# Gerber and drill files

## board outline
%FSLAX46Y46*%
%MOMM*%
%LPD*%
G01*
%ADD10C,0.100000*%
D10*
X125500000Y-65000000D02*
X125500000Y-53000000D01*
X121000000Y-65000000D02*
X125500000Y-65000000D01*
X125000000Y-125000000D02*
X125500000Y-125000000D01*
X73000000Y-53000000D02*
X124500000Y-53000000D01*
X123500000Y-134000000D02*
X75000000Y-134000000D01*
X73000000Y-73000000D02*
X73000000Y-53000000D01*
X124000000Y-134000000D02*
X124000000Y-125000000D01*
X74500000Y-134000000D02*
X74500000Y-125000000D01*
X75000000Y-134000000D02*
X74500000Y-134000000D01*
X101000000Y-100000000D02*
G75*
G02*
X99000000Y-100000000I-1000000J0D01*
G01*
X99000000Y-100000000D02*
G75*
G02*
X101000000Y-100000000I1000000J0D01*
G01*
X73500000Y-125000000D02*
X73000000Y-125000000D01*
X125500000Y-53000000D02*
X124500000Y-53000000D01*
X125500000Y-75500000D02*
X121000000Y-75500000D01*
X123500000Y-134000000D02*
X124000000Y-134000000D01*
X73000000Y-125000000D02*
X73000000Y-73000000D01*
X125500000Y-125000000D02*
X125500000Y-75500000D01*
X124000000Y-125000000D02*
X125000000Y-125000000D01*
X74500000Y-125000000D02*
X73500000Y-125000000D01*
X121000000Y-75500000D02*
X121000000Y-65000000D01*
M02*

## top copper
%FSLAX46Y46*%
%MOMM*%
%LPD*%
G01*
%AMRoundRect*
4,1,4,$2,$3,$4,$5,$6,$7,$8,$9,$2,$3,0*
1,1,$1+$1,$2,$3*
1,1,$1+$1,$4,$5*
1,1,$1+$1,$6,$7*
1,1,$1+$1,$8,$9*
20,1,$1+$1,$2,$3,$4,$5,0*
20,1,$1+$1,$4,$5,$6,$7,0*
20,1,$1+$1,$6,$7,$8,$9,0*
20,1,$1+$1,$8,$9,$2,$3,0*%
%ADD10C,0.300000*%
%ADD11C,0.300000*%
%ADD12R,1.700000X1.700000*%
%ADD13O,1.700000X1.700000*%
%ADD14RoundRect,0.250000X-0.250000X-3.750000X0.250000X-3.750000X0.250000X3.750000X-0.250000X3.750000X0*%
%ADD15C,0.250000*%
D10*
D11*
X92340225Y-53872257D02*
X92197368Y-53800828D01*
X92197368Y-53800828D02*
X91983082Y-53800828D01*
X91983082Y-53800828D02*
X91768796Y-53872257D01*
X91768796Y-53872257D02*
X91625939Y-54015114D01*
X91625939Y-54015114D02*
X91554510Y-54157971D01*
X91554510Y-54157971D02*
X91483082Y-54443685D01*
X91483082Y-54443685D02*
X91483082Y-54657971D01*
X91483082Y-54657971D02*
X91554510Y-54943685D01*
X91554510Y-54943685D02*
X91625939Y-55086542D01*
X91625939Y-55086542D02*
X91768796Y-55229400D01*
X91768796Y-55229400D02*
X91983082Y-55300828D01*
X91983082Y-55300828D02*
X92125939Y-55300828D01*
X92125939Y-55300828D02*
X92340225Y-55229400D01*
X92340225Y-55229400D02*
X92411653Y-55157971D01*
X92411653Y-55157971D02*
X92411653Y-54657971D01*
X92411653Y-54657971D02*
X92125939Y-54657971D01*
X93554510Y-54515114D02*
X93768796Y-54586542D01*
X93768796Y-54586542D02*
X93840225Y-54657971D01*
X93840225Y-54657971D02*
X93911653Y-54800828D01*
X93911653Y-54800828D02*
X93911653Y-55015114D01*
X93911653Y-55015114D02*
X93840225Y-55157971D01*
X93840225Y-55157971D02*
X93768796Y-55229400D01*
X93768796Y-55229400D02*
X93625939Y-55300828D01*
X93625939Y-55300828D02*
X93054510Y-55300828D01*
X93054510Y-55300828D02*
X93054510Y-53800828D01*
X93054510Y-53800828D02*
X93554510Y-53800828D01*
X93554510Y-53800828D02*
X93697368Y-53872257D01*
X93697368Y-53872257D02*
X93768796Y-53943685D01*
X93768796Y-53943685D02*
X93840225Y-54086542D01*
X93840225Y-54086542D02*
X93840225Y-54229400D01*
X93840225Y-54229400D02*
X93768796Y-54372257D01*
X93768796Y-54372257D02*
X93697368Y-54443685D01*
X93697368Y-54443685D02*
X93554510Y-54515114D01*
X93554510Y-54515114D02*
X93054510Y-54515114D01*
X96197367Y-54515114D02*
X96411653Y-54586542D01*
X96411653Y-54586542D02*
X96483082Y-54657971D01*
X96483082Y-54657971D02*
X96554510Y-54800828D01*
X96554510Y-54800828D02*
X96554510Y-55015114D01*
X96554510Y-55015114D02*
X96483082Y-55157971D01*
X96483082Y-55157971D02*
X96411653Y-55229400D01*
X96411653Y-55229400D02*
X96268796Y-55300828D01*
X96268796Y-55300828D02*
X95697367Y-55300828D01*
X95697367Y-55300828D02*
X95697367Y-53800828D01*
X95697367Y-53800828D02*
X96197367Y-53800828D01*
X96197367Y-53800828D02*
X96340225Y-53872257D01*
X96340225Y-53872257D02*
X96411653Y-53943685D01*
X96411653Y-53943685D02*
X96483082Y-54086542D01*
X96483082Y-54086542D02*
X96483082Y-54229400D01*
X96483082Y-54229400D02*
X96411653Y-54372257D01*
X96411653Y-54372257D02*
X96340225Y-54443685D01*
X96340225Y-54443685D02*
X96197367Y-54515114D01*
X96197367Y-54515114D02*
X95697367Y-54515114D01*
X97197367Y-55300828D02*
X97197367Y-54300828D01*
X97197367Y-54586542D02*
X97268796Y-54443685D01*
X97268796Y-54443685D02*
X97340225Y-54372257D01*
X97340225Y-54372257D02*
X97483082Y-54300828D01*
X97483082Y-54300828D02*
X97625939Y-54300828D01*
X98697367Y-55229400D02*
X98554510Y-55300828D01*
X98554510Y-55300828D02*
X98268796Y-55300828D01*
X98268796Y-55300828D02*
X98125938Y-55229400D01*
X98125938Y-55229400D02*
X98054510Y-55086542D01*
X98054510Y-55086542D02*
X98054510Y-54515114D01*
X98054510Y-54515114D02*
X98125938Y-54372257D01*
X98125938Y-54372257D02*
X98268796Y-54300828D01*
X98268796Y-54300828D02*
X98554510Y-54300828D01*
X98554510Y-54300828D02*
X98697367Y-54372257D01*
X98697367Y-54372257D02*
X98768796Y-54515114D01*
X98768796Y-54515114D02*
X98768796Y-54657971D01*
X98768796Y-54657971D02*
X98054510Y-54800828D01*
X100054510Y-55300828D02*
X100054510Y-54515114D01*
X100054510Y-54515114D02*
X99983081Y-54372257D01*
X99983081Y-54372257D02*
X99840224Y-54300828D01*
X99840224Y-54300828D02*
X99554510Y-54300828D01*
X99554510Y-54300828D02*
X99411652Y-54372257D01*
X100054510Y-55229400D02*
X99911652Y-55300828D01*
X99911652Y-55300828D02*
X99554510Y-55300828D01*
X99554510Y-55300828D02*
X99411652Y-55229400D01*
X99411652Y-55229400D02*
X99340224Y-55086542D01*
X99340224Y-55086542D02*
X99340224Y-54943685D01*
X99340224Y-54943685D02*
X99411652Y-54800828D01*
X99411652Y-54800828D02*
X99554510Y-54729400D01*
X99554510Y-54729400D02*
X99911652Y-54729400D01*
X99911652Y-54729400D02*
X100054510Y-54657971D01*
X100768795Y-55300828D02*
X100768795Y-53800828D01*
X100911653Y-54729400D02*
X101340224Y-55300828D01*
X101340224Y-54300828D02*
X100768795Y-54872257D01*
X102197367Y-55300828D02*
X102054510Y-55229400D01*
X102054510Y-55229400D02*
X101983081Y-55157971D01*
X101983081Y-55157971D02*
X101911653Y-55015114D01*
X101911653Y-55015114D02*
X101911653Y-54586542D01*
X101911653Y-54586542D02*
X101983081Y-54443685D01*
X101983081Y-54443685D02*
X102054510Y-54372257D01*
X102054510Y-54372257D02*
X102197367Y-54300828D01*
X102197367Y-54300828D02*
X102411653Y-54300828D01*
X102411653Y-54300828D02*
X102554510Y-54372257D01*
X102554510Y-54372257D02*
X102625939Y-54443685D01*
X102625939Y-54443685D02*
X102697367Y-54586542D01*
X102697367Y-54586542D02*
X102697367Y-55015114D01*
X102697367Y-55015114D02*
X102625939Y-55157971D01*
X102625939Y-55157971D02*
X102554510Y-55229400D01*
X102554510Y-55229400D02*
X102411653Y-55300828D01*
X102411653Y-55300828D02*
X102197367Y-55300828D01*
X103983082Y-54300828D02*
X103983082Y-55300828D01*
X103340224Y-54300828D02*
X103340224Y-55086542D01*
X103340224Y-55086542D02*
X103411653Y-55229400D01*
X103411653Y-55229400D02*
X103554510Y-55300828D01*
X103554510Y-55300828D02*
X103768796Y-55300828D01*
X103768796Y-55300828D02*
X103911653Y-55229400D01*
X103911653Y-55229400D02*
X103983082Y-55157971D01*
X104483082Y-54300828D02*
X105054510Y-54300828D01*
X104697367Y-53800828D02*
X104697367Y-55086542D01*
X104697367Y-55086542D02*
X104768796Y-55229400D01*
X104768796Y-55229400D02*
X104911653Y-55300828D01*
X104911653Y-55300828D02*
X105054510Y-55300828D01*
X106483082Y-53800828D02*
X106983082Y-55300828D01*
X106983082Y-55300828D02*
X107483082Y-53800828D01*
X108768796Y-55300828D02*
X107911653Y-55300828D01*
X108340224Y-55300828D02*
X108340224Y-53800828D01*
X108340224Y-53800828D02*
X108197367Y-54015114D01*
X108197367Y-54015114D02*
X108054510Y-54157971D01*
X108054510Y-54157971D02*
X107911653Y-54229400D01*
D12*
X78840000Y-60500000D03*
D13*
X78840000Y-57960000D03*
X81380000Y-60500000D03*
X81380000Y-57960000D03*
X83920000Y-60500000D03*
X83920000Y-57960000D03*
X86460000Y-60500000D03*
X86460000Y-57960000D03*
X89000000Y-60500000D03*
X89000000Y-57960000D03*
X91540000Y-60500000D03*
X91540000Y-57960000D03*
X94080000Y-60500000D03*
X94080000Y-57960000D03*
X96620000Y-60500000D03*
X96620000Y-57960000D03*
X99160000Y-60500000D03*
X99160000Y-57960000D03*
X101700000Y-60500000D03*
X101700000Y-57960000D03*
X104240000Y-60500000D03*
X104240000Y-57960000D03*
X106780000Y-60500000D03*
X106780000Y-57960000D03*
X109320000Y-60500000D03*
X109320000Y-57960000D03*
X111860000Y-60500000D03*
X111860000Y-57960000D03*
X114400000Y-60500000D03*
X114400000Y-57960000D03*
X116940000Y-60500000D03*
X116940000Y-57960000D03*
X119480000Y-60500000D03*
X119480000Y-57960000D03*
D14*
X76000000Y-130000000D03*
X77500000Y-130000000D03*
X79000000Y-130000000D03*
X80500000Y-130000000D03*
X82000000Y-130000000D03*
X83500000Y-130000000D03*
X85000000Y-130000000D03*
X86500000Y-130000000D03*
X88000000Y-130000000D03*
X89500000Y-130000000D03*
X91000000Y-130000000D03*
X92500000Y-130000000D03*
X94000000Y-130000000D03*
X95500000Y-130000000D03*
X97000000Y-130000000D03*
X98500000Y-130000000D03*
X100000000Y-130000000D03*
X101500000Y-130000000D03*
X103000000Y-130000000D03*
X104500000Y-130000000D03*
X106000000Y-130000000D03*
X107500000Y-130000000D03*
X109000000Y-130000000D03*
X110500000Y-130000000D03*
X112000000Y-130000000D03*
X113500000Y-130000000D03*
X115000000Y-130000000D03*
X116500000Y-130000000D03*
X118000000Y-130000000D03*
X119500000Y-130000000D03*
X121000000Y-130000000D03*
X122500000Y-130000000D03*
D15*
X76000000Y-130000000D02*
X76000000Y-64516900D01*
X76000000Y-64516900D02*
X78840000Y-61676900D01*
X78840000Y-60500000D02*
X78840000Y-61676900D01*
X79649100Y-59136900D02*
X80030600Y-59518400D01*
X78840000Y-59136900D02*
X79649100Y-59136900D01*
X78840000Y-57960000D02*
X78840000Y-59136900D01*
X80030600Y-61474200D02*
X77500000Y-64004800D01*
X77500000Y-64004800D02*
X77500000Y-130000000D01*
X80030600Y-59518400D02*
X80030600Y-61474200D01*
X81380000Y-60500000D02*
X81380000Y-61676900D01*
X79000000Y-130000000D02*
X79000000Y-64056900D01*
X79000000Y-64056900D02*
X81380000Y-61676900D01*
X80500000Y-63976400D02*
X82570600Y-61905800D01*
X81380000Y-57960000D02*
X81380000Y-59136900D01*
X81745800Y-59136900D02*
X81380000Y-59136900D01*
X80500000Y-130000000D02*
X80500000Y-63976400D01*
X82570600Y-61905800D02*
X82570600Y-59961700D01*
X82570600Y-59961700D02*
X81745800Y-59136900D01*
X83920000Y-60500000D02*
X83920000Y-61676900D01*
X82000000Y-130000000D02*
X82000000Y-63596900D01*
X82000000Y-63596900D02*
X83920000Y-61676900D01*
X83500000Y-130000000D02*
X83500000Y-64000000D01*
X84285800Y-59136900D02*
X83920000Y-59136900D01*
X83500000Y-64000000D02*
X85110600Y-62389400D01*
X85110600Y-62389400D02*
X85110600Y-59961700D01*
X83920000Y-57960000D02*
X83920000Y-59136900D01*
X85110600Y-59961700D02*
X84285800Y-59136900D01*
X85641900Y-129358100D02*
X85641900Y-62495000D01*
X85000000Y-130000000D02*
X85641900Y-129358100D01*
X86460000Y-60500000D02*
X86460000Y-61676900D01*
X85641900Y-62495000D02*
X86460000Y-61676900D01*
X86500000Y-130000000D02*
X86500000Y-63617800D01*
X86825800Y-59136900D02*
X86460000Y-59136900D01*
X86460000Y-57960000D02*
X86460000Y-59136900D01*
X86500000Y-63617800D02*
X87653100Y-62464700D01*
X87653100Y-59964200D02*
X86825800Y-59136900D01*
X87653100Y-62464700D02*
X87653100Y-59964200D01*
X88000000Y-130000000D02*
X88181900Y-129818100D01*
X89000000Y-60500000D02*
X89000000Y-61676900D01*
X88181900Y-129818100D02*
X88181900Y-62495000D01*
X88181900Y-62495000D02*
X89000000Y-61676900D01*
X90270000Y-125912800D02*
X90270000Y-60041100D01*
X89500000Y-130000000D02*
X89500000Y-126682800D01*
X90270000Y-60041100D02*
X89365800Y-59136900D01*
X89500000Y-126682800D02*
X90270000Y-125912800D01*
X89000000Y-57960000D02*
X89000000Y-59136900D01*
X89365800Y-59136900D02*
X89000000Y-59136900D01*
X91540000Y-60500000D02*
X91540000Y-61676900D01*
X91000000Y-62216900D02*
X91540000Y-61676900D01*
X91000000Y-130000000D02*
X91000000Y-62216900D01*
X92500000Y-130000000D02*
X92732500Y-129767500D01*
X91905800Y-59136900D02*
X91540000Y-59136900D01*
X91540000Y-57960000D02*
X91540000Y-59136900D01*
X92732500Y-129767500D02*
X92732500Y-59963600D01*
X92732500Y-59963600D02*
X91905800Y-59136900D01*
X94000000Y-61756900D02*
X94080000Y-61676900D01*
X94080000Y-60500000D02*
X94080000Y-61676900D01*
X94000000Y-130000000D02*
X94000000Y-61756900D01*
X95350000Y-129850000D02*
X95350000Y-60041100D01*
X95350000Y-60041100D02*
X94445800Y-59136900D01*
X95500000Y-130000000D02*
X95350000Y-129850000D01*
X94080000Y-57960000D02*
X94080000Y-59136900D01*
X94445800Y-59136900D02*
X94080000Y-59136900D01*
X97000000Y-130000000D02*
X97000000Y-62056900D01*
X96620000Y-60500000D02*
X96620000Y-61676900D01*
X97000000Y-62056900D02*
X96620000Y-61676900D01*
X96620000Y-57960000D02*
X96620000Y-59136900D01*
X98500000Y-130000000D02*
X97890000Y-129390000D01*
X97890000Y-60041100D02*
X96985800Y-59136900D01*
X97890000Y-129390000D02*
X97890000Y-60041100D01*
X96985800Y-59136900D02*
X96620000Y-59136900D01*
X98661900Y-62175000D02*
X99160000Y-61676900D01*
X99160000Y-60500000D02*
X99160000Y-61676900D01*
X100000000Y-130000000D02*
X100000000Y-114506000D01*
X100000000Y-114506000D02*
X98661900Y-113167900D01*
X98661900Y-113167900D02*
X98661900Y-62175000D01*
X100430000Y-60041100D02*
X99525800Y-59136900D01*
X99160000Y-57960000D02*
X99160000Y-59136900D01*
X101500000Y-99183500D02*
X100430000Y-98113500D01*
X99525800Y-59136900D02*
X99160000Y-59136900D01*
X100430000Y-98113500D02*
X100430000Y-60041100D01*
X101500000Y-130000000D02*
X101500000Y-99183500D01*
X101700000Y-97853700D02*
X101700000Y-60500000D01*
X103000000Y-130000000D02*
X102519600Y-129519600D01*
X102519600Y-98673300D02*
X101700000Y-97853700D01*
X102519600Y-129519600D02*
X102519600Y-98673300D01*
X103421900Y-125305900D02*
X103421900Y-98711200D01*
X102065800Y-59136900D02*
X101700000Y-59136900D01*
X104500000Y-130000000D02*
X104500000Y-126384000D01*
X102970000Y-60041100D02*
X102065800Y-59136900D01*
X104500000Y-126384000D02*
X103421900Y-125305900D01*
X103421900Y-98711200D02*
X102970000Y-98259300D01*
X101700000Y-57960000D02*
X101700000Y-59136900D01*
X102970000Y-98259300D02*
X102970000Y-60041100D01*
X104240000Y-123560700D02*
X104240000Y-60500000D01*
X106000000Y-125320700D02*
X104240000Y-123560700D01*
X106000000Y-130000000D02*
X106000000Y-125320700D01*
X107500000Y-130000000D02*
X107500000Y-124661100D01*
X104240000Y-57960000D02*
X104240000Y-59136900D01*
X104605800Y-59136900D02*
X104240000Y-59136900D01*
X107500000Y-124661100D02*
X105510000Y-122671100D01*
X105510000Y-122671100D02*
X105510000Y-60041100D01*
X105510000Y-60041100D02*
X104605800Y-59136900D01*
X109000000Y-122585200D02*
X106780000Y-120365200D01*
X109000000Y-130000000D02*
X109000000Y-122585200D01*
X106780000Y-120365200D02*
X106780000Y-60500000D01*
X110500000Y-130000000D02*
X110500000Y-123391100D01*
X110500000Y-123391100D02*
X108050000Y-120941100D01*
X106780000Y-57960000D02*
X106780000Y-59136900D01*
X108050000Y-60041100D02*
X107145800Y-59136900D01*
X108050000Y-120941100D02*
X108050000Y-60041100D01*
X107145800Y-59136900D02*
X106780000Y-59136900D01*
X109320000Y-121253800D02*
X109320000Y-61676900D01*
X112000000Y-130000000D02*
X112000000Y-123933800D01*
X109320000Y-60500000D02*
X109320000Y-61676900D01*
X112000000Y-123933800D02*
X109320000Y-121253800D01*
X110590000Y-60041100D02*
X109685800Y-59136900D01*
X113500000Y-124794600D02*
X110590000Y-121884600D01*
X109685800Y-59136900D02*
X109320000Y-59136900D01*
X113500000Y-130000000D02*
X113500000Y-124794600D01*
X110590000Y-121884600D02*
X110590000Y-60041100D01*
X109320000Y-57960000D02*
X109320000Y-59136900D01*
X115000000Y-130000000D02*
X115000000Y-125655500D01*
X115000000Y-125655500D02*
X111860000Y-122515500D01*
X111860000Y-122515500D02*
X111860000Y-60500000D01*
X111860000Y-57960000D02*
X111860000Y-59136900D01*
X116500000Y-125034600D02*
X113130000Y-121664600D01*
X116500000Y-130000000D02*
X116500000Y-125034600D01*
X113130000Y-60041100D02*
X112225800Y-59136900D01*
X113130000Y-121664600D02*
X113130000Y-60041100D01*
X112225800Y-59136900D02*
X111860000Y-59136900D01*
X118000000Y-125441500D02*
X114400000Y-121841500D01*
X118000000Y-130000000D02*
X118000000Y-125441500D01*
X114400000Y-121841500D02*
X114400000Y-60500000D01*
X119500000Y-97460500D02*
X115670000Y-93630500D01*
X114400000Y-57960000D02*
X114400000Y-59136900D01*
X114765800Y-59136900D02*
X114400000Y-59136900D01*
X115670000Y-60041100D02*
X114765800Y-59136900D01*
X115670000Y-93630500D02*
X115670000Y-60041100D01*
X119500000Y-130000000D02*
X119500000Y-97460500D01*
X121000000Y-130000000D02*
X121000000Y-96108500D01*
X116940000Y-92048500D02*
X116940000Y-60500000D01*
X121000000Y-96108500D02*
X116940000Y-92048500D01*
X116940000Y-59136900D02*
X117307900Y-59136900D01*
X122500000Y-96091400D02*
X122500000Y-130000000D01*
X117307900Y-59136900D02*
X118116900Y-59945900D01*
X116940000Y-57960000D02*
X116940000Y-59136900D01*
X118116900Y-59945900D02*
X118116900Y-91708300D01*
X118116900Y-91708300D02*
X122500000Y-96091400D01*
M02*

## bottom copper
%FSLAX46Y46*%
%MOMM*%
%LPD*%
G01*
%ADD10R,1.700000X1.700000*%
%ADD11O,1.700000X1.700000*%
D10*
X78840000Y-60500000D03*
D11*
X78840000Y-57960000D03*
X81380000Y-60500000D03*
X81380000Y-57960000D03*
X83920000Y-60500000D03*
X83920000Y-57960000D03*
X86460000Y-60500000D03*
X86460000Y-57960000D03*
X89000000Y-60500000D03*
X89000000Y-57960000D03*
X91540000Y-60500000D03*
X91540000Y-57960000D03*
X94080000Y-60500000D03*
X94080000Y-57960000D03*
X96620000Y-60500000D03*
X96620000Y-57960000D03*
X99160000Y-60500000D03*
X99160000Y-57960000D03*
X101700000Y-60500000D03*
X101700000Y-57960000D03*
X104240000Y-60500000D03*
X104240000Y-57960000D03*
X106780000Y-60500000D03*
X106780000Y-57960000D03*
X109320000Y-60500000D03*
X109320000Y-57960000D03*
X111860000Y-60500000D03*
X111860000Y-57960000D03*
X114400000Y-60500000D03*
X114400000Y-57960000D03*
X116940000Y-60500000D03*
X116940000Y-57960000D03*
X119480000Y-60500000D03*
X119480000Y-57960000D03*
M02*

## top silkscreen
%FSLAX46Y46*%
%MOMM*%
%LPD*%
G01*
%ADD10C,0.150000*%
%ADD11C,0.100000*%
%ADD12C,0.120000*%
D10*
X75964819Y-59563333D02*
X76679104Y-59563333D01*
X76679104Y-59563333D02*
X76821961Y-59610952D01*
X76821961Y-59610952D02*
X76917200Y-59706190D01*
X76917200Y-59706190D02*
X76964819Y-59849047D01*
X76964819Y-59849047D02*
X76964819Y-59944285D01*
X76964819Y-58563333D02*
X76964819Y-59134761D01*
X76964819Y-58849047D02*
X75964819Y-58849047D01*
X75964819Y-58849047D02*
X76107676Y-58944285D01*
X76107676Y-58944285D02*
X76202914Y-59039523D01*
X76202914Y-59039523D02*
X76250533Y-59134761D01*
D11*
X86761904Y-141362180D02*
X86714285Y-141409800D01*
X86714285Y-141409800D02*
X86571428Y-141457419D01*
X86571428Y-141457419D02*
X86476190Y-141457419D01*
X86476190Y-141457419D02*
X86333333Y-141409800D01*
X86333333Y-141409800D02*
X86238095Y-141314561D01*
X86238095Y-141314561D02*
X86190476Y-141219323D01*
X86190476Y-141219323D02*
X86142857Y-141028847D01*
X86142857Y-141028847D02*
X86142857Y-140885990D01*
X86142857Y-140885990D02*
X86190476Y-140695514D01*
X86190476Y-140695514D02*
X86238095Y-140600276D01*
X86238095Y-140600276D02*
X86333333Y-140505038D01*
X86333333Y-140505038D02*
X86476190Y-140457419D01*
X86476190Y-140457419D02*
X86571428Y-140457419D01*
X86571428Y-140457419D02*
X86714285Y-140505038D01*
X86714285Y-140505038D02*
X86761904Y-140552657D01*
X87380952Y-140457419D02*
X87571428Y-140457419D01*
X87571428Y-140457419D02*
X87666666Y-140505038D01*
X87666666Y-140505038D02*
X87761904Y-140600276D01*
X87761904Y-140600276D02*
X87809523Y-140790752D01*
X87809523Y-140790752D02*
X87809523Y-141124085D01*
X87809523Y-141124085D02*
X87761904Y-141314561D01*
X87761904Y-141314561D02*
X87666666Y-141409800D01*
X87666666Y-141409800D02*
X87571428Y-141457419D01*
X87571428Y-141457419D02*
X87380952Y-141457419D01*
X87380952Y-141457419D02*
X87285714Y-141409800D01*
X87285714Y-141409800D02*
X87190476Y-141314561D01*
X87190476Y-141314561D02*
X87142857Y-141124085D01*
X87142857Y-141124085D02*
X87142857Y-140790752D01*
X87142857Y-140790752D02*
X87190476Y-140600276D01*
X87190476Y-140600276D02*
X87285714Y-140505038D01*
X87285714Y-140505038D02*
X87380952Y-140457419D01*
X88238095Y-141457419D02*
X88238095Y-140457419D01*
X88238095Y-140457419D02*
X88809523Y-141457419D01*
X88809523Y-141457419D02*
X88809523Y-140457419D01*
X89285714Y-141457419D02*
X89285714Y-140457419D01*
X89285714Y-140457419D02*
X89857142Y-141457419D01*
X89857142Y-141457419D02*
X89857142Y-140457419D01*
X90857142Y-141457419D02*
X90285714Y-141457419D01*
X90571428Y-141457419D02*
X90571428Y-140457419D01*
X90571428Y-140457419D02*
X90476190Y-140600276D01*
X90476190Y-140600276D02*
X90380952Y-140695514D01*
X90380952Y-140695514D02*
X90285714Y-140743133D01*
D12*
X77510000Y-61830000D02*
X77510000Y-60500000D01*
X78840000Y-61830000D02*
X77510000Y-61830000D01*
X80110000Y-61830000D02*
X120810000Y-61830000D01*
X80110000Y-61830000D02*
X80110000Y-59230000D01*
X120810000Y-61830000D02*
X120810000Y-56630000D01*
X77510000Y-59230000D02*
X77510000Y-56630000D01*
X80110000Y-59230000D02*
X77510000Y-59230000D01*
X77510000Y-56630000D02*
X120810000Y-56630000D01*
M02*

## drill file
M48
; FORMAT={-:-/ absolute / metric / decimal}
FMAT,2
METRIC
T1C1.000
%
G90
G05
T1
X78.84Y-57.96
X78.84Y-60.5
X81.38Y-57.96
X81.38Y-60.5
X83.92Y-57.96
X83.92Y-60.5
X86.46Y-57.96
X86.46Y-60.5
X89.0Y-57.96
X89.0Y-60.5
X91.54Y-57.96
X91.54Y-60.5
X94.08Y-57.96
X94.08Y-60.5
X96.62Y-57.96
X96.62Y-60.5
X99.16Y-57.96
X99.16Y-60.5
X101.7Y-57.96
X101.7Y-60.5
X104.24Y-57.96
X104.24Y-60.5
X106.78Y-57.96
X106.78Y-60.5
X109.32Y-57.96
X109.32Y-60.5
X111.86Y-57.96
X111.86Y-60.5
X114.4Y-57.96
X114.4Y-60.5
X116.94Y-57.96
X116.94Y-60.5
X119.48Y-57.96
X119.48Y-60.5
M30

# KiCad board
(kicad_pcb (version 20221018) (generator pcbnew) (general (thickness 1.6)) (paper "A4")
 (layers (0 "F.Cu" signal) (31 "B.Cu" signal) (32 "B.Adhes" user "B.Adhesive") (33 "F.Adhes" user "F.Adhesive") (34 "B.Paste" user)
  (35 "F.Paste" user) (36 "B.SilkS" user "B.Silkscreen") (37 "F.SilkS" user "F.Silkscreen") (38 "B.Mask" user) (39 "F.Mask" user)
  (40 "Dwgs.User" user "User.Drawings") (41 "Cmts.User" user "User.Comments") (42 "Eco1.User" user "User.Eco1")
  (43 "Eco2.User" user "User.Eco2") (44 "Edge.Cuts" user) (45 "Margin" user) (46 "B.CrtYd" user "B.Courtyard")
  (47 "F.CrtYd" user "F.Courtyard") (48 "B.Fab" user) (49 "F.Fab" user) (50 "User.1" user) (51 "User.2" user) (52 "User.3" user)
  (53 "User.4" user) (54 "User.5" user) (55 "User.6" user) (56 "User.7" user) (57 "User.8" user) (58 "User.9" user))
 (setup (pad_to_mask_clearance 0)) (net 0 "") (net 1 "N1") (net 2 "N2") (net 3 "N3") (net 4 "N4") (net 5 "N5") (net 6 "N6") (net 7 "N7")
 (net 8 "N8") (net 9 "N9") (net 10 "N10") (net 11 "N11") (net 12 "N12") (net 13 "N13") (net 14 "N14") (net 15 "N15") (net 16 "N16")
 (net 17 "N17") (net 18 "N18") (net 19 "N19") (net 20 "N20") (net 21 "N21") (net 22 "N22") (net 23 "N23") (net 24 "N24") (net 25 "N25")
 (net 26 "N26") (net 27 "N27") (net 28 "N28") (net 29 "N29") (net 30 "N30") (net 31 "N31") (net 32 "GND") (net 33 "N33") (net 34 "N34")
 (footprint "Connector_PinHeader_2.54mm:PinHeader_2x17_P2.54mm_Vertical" (layer "F.Cu") (at 78.84 60.5 90)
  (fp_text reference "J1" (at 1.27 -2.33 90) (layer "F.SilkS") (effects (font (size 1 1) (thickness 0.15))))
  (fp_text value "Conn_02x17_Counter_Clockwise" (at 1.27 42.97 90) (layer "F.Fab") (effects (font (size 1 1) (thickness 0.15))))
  (fp_line (start -1.33 -1.33) (end 0 -1.33) (stroke (width 0.12) (type solid)) (layer "F.SilkS"))
  (fp_line (start -1.33 0) (end -1.33 -1.33) (stroke (width 0.12) (type solid)) (layer "F.SilkS"))
  (fp_line (start -1.33 1.27) (end -1.33 41.97) (stroke (width 0.12) (type solid)) (layer "F.SilkS"))
  (fp_line (start -1.33 1.27) (end 1.27 1.27) (stroke (width 0.12) (type solid)) (layer "F.SilkS"))
  (fp_line (start -1.33 41.97) (end 3.87 41.97) (stroke (width 0.12) (type solid)) (layer "F.SilkS"))
  (fp_line (start 1.27 -1.33) (end 3.87 -1.33) (stroke (width 0.12) (type solid)) (layer "F.SilkS"))
  (fp_line (start 1.27 1.27) (end 1.27 -1.33) (stroke (width 0.12) (type solid)) (layer "F.SilkS"))
  (fp_line (start 3.87 -1.33) (end 3.87 41.97) (stroke (width 0.12) (type solid)) (layer "F.SilkS"))
  (pad "1" thru_hole rect (at 0 0 90) (size 1.7 1.7) (drill 1) (layers "*.Cu" "*.Mask") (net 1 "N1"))
  (pad "2" thru_hole oval (at 2.54 0 90) (size 1.7 1.7) (drill 1) (layers "*.Cu" "*.Mask") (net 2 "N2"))
  (pad "3" thru_hole oval (at 0 2.54 90) (size 1.7 1.7) (drill 1) (layers "*.Cu" "*.Mask") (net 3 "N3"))
  (pad "4" thru_hole oval (at 2.54 2.54 90) (size 1.7 1.7) (drill 1) (layers "*.Cu" "*.Mask") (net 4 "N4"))
  (pad "5" thru_hole oval (at 0 5.08 90) (size 1.7 1.7) (drill 1) (layers "*.Cu" "*.Mask") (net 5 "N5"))
  (pad "6" thru_hole oval (at 2.54 5.08 90) (size 1.7 1.7) (drill 1) (layers "*.Cu" "*.Mask") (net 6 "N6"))
  (pad "7" thru_hole oval (at 0 7.62 90) (size 1.7 1.7) (drill 1) (layers "*.Cu" "*.Mask") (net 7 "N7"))
  (pad "8" thru_hole oval (at 2.54 7.62 90) (size 1.7 1.7) (drill 1) (layers "*.Cu" "*.Mask") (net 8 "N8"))
  (pad "9" thru_hole oval (at 0 10.16 90) (size 1.7 1.7) (drill 1) (layers "*.Cu" "*.Mask") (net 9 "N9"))
  (pad "10" thru_hole oval (at 2.54 10.16 90) (size 1.7 1.7) (drill 1) (layers "*.Cu" "*.Mask") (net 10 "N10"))
  (pad "11" thru_hole oval (at 0 12.7 90) (size 1.7 1.7) (drill 1) (layers "*.Cu" "*.Mask") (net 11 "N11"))
  (pad "12" thru_hole oval (at 2.54 12.7 90) (size 1.7 1.7) (drill 1) (layers "*.Cu" "*.Mask") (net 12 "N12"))
  (pad "13" thru_hole oval (at 0 15.24 90) (size 1.7 1.7) (drill 1) (layers "*.Cu" "*.Mask") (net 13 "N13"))
  (pad "14" thru_hole oval (at 2.54 15.24 90) (size 1.7 1.7) (drill 1) (layers "*.Cu" "*.Mask") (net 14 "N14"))
  (pad "15" thru_hole oval (at 0 17.78 90) (size 1.7 1.7) (drill 1) (layers "*.Cu" "*.Mask") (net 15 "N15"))
  (pad "16" thru_hole oval (at 2.54 17.78 90) (size 1.7 1.7) (drill 1) (layers "*.Cu" "*.Mask") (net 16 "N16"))
  (pad "17" thru_hole oval (at 0 20.32 90) (size 1.7 1.7) (drill 1) (layers "*.Cu" "*.Mask") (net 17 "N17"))
  (pad "18" thru_hole oval (at 2.54 20.32 90) (size 1.7 1.7) (drill 1) (layers "*.Cu" "*.Mask") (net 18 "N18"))
  (pad "19" thru_hole oval (at 0 22.86 90) (size 1.7 1.7) (drill 1) (layers "*.Cu" "*.Mask") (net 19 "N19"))
  (pad "20" thru_hole oval (at 2.54 22.86 90) (size 1.7 1.7) (drill 1) (layers "*.Cu" "*.Mask") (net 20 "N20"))
  (pad "21" thru_hole oval (at 0 25.4 90) (size 1.7 1.7) (drill 1) (layers "*.Cu" "*.Mask") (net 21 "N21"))
  (pad "22" thru_hole oval (at 2.54 25.4 90) (size 1.7 1.7) (drill 1) (layers "*.Cu" "*.Mask") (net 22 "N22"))
  (pad "23" thru_hole oval (at 0 27.94 90) (size 1.7 1.7) (drill 1) (layers "*.Cu" "*.Mask") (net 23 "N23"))
  (pad "24" thru_hole oval (at 2.54 27.94 90) (size 1.7 1.7) (drill 1) (layers "*.Cu" "*.Mask") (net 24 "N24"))
  (pad "25" thru_hole oval (at 0 30.48 90) (size 1.7 1.7) (drill 1) (layers "*.Cu" "*.Mask") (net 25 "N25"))
  (pad "26" thru_hole oval (at 2.54 30.48 90) (size 1.7 1.7) (drill 1) (layers "*.Cu" "*.Mask") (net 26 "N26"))
  (pad "27" thru_hole oval (at 0 33.02 90) (size 1.7 1.7) (drill 1) (layers "*.Cu" "*.Mask") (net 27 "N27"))
  (pad "28" thru_hole oval (at 2.54 33.02 90) (size 1.7 1.7) (drill 1) (layers "*.Cu" "*.Mask") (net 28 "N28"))
  (pad "29" thru_hole oval (at 0 35.56 90) (size 1.7 1.7) (drill 1) (layers "*.Cu" "*.Mask") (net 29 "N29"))
  (pad "30" thru_hole oval (at 2.54 35.56 90) (size 1.7 1.7) (drill 1) (layers "*.Cu" "*.Mask") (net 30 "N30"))
  (pad "31" thru_hole oval (at 0 38.1 90) (size 1.7 1.7) (drill 1) (layers "*.Cu" "*.Mask") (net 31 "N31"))
  (pad "32" thru_hole oval (at 2.54 38.1 90) (size 1.7 1.7) (drill 1) (layers "*.Cu" "*.Mask") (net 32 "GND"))
  (pad "33" thru_hole oval (at 0 40.64 90) (size 1.7 1.7) (drill 1) (layers "*.Cu" "*.Mask") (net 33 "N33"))
  (pad "34" thru_hole oval (at 2.54 40.64 90) (size 1.7 1.7) (drill 1) (layers "*.Cu" "*.Mask") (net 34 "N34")))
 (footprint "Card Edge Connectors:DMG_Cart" (layer "F.Cu") (at 75 134)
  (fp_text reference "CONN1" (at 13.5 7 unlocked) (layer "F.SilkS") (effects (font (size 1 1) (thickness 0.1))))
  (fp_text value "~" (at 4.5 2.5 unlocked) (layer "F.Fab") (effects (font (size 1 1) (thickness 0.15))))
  (pad "1" smd roundrect (at 1 -4) (size 1 8) (layers "F.Cu" "F.Paste" "F.Mask") (roundrect_rratio 0.25) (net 1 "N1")
   (thermal_bridge_angle 45))
  (pad "2" smd roundrect (at 2.5 -4) (size 1 8) (layers "F.Cu" "F.Paste" "F.Mask") (roundrect_rratio 0.25) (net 2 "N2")
   (thermal_bridge_angle 45))
  (pad "3" smd roundrect (at 4 -4) (size 1 8) (layers "F.Cu" "F.Paste" "F.Mask") (roundrect_rratio 0.25) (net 3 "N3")
   (thermal_bridge_angle 45))
  (pad "4" smd roundrect (at 5.5 -4) (size 1 8) (layers "F.Cu" "F.Paste" "F.Mask") (roundrect_rratio 0.25) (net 4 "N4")
   (thermal_bridge_angle 45))
  (pad "5" smd roundrect (at 7 -4) (size 1 8) (layers "F.Cu" "F.Paste" "F.Mask") (roundrect_rratio 0.25) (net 5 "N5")
   (thermal_bridge_angle 45))
  (pad "6" smd roundrect (at 8.5 -4) (size 1 8) (layers "F.Cu" "F.Paste" "F.Mask") (roundrect_rratio 0.25) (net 6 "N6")
   (thermal_bridge_angle 45))
  (pad "7" smd roundrect (at 10 -4) (size 1 8) (layers "F.Cu" "F.Paste" "F.Mask") (roundrect_rratio 0.25) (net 7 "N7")
   (thermal_bridge_angle 45))
  (pad "8" smd roundrect (at 11.5 -4) (size 1 8) (layers "F.Cu" "F.Paste" "F.Mask") (roundrect_rratio 0.25) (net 8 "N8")
   (thermal_bridge_angle 45))
  (pad "9" smd roundrect (at 13 -4) (size 1 8) (layers "F.Cu" "F.Paste" "F.Mask") (roundrect_rratio 0.25) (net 9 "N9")
   (thermal_bridge_angle 45))
  (pad "10" smd roundrect (at 14.5 -4) (size 1 8) (layers "F.Cu" "F.Paste" "F.Mask") (roundrect_rratio 0.25) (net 10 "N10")
   (thermal_bridge_angle 45))
  (pad "11" smd roundrect (at 16 -4) (size 1 8) (layers "F.Cu" "F.Paste" "F.Mask") (roundrect_rratio 0.25) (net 11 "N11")
   (thermal_bridge_angle 45))
  (pad "12" smd roundrect (at 17.5 -4) (size 1 8) (layers "F.Cu" "F.Paste" "F.Mask") (roundrect_rratio 0.25) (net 12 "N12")
   (thermal_bridge_angle 45))
  (pad "13" smd roundrect (at 19 -4) (size 1 8) (layers "F.Cu" "F.Paste" "F.Mask") (roundrect_rratio 0.25) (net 13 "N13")
   (thermal_bridge_angle 45))
  (pad "14" smd roundrect (at 20.5 -4) (size 1 8) (layers "F.Cu" "F.Paste" "F.Mask") (roundrect_rratio 0.25) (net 14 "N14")
   (thermal_bridge_angle 45))
  (pad "15" smd roundrect (at 22 -4) (size 1 8) (layers "F.Cu" "F.Paste" "F.Mask") (roundrect_rratio 0.25) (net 15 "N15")
   (thermal_bridge_angle 45))
  (pad "16" smd roundrect (at 23.5 -4) (size 1 8) (layers "F.Cu" "F.Paste" "F.Mask") (roundrect_rratio 0.25) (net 16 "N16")
   (thermal_bridge_angle 45))
  (pad "17" smd roundrect (at 25 -4) (size 1 8) (layers "F.Cu" "F.Paste" "F.Mask") (roundrect_rratio 0.25) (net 17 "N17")
   (thermal_bridge_angle 45))
  (pad "18" smd roundrect (at 26.5 -4) (size 1 8) (layers "F.Cu" "F.Paste" "F.Mask") (roundrect_rratio 0.25) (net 18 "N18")
   (thermal_bridge_angle 45))
  (pad "19" smd roundrect (at 28 -4) (size 1 8) (layers "F.Cu" "F.Paste" "F.Mask") (roundrect_rratio 0.25) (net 19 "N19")
   (thermal_bridge_angle 45))
  (pad "20" smd roundrect (at 29.5 -4) (size 1 8) (layers "F.Cu" "F.Paste" "F.Mask") (roundrect_rratio 0.25) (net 20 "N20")
   (thermal_bridge_angle 45))
  (pad "21" smd roundrect (at 31 -4) (size 1 8) (layers "F.Cu" "F.Paste" "F.Mask") (roundrect_rratio 0.25) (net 21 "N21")
   (thermal_bridge_angle 45))
  (pad "22" smd roundrect (at 32.5 -4) (size 1 8) (layers "F.Cu" "F.Paste" "F.Mask") (roundrect_rratio 0.25) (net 22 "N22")
   (thermal_bridge_angle 45))
  (pad "23" smd roundrect (at 34 -4) (size 1 8) (layers "F.Cu" "F.Paste" "F.Mask") (roundrect_rratio 0.25) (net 23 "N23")
   (thermal_bridge_angle 45))
  (pad "24" smd roundrect (at 35.5 -4) (size 1 8) (layers "F.Cu" "F.Paste" "F.Mask") (roundrect_rratio 0.25) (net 24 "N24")
   (thermal_bridge_angle 45))
  (pad "25" smd roundrect (at 37 -4) (size 1 8) (layers "F.Cu" "F.Paste" "F.Mask") (roundrect_rratio 0.25) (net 25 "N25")
   (thermal_bridge_angle 45))
  (pad "26" smd roundrect (at 38.5 -4) (size 1 8) (layers "F.Cu" "F.Paste" "F.Mask") (roundrect_rratio 0.25) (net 26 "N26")
   (thermal_bridge_angle 45))
  (pad "27" smd roundrect (at 40 -4) (size 1 8) (layers "F.Cu" "F.Paste" "F.Mask") (roundrect_rratio 0.25) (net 27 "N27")
   (thermal_bridge_angle 45))
  (pad "28" smd roundrect (at 41.5 -4) (size 1 8) (layers "F.Cu" "F.Paste" "F.Mask") (roundrect_rratio 0.25) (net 28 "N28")
   (thermal_bridge_angle 45))
  (pad "29" smd roundrect (at 43 -4) (size 1 8) (layers "F.Cu" "F.Paste" "F.Mask") (roundrect_rratio 0.25) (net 29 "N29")
   (thermal_bridge_angle 45))
  (pad "30" smd roundrect (at 44.5 -4) (size 1 8) (layers "F.Cu" "F.Paste" "F.Mask") (roundrect_rratio 0.25) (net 30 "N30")
   (thermal_bridge_angle 45))
  (pad "31" smd roundrect (at 46 -4) (size 1 8) (layers "F.Cu" "F.Paste" "F.Mask") (roundrect_rratio 0.25) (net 31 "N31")
   (thermal_bridge_angle 45))
  (pad "32" smd roundrect (at 47.5 -4) (size 1 8) (layers "F.Cu" "F.Paste" "F.Mask") (roundrect_rratio 0.25) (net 32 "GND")
   (thermal_bridge_angle 45)))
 (gr_line (start 125.5 65) (end 125.5 53) (stroke (width 0.1) (type default)) (layer "Edge.Cuts"))
 (gr_line (start 121 65) (end 125.5 65) (stroke (width 0.1) (type default)) (layer "Edge.Cuts"))
 (gr_line (start 125 125) (end 125.5 125) (stroke (width 0.1) (type default)) (layer "Edge.Cuts"))
 (gr_line (start 73 53) (end 124.5 53) (stroke (width 0.1) (type default)) (layer "Edge.Cuts"))
 (gr_line (start 123.5 134) (end 75 134) (stroke (width 0.1) (type default)) (layer "Edge.Cuts"))
 (gr_line (start 73 73) (end 73 53) (stroke (width 0.1) (type default)) (layer "Edge.Cuts"))
 (gr_line (start 124 134) (end 124 125) (stroke (width 0.1) (type default)) (layer "Edge.Cuts"))
 (gr_line (start 74.5 134) (end 74.5 125) (stroke (width 0.1) (type default)) (layer "Edge.Cuts"))
 (gr_line (start 75 134) (end 74.5 134) (stroke (width 0.1) (type default)) (layer "Edge.Cuts"))
 (gr_circle (center 100 100) (end 101 100) (stroke (width 0.1) (type default)) (fill none) (layer "Edge.Cuts"))
 (gr_line (start 73.5 125) (end 73 125) (stroke (width 0.1) (type default)) (layer "Edge.Cuts"))
 (gr_line (start 125.5 53) (end 124.5 53) (stroke (width 0.1) (type default)) (layer "Edge.Cuts"))
 (gr_line (start 125.5 75.5) (end 121 75.5) (stroke (width 0.1) (type default)) (layer "Edge.Cuts"))
 (gr_line (start 123.5 134) (end 124 134) (stroke (width 0.1) (type default)) (layer "Edge.Cuts"))
 (gr_line (start 73 125) (end 73 73) (stroke (width 0.1) (type default)) (layer "Edge.Cuts"))
 (gr_line (start 125.5 125) (end 125.5 75.5) (stroke (width 0.1) (type default)) (layer "Edge.Cuts"))
 (gr_line (start 124 125) (end 125 125) (stroke (width 0.1) (type default)) (layer "Edge.Cuts"))
 (gr_line (start 74.5 125) (end 73.5 125) (stroke (width 0.1) (type default)) (layer "Edge.Cuts"))
 (gr_line (start 121 75.5) (end 121 65) (stroke (width 0.1) (type default)) (layer "Edge.Cuts"))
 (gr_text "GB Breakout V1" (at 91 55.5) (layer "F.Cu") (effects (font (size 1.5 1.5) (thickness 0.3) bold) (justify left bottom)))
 (segment (start 76 130) (end 76 64.5169) (width 0.25) (layer "F.Cu") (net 1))
 (segment (start 76 64.5169) (end 78.84 61.6769) (width 0.25) (layer "F.Cu") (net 1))
 (segment (start 78.84 60.5) (end 78.84 61.6769) (width 0.25) (layer "F.Cu") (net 1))
 (segment (start 79.6491 59.1369) (end 80.0306 59.5184) (width 0.25) (layer "F.Cu") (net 2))
 (segment (start 78.84 59.1369) (end 79.6491 59.1369) (width 0.25) (layer "F.Cu") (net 2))
 (segment (start 78.84 57.96) (end 78.84 59.1369) (width 0.25) (layer "F.Cu") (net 2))
 (segment (start 80.0306 61.4742) (end 77.5 64.0048) (width 0.25) (layer "F.Cu") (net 2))
 (segment (start 77.5 64.0048) (end 77.5 130) (width 0.25) (layer "F.Cu") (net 2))
 (segment (start 80.0306 59.5184) (end 80.0306 61.4742) (width 0.25) (layer "F.Cu") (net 2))
 (segment (start 81.38 60.5) (end 81.38 61.6769) (width 0.25) (layer "F.Cu") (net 3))
 (segment (start 79 130) (end 79 64.0569) (width 0.25) (layer "F.Cu") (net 3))
 (segment (start 79 64.0569) (end 81.38 61.6769) (width 0.25) (layer "F.Cu") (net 3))
 (segment (start 80.5 63.9764) (end 82.5706 61.9058) (width 0.25) (layer "F.Cu") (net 4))
 (segment (start 81.38 57.96) (end 81.38 59.1369) (width 0.25) (layer "F.Cu") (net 4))
 (segment (start 81.7458 59.1369) (end 81.38 59.1369) (width 0.25) (layer "F.Cu") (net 4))
 (segment (start 80.5 130) (end 80.5 63.9764) (width 0.25) (layer "F.Cu") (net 4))
 (segment (start 82.5706 61.9058) (end 82.5706 59.9617) (width 0.25) (layer "F.Cu") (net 4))
 (segment (start 82.5706 59.9617) (end 81.7458 59.1369) (width 0.25) (layer "F.Cu") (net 4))
 (segment (start 83.92 60.5) (end 83.92 61.6769) (width 0.25) (layer "F.Cu") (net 5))
 (segment (start 82 130) (end 82 63.5969) (width 0.25) (layer "F.Cu") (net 5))
 (segment (start 82 63.5969) (end 83.92 61.6769) (width 0.25) (layer "F.Cu") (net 5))
 (segment (start 83.5 130) (end 83.5 64) (width 0.25) (layer "F.Cu") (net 6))
 (segment (start 84.2858 59.1369) (end 83.92 59.1369) (width 0.25) (layer "F.Cu") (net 6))
 (segment (start 83.5 64) (end 85.1106 62.3894) (width 0.25) (layer "F.Cu") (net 6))
 (segment (start 85.1106 62.3894) (end 85.1106 59.9617) (width 0.25) (layer "F.Cu") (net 6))
 (segment (start 83.92 57.96) (end 83.92 59.1369) (width 0.25) (layer "F.Cu") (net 6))
 (segment (start 85.1106 59.9617) (end 84.2858 59.1369) (width 0.25) (layer "F.Cu") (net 6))
 (segment (start 85.6419 129.3581) (end 85.6419 62.495) (width 0.25) (layer "F.Cu") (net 7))
 (segment (start 85 130) (end 85.6419 129.3581) (width 0.25) (layer "F.Cu") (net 7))
 (segment (start 86.46 60.5) (end 86.46 61.6769) (width 0.25) (layer "F.Cu") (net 7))
 (segment (start 85.6419 62.495) (end 86.46 61.6769) (width 0.25) (layer "F.Cu") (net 7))
 (segment (start 86.5 130) (end 86.5 63.6178) (width 0.25) (layer "F.Cu") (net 8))
 (segment (start 86.8258 59.1369) (end 86.46 59.1369) (width 0.25) (layer "F.Cu") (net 8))
 (segment (start 86.46 57.96) (end 86.46 59.1369) (width 0.25) (layer "F.Cu") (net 8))
 (segment (start 86.5 63.6178) (end 87.6531 62.4647) (width 0.25) (layer "F.Cu") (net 8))
 (segment (start 87.6531 59.9642) (end 86.8258 59.1369) (width 0.25) (layer "F.Cu") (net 8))
 (segment (start 87.6531 62.4647) (end 87.6531 59.9642) (width 0.25) (layer "F.Cu") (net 8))
 (segment (start 88 130) (end 88.1819 129.8181) (width 0.25) (layer "F.Cu") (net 9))
 (segment (start 89 60.5) (end 89 61.6769) (width 0.25) (layer "F.Cu") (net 9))
 (segment (start 88.1819 129.8181) (end 88.1819 62.495) (width 0.25) (layer "F.Cu") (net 9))
 (segment (start 88.1819 62.495) (end 89 61.6769) (width 0.25) (layer "F.Cu") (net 9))
 (segment (start 90.27 125.9128) (end 90.27 60.0411) (width 0.25) (layer "F.Cu") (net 10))
 (segment (start 89.5 130) (end 89.5 126.6828) (width 0.25) (layer "F.Cu") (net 10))
 (segment (start 90.27 60.0411) (end 89.3658 59.1369) (width 0.25) (layer "F.Cu") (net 10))
 (segment (start 89.5 126.6828) (end 90.27 125.9128) (width 0.25) (layer "F.Cu") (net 10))
 (segment (start 89 57.96) (end 89 59.1369) (width 0.25) (layer "F.Cu") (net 10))
 (segment (start 89.3658 59.1369) (end 89 59.1369) (width 0.25) (layer "F.Cu") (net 10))
 (segment (start 91.54 60.5) (end 91.54 61.6769) (width 0.25) (layer "F.Cu") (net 11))
 (segment (start 91 62.2169) (end 91.54 61.6769) (width 0.25) (layer "F.Cu") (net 11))
 (segment (start 91 130) (end 91 62.2169) (width 0.25) (layer "F.Cu") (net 11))
 (segment (start 92.5 130) (end 92.7325 129.7675) (width 0.25) (layer "F.Cu") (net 12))
 (segment (start 91.9058 59.1369) (end 91.54 59.1369) (width 0.25) (layer "F.Cu") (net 12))
 (segment (start 91.54 57.96) (end 91.54 59.1369) (width 0.25) (layer "F.Cu") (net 12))
 (segment (start 92.7325 129.7675) (end 92.7325 59.9636) (width 0.25) (layer "F.Cu") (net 12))
 (segment (start 92.7325 59.9636) (end 91.9058 59.1369) (width 0.25) (layer "F.Cu") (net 12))
 (segment (start 94 61.7569) (end 94.08 61.6769) (width 0.25) (layer "F.Cu") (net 13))
 (segment (start 94.08 60.5) (end 94.08 61.6769) (width 0.25) (layer "F.Cu") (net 13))
 (segment (start 94 130) (end 94 61.7569) (width 0.25) (layer "F.Cu") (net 13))
 (segment (start 95.35 129.85) (end 95.35 60.0411) (width 0.25) (layer "F.Cu") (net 14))
 (segment (start 95.35 60.0411) (end 94.4458 59.1369) (width 0.25) (layer "F.Cu") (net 14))
 (segment (start 95.5 130) (end 95.35 129.85) (width 0.25) (layer "F.Cu") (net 14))
 (segment (start 94.08 57.96) (end 94.08 59.1369) (width 0.25) (layer "F.Cu") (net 14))
 (segment (start 94.4458 59.1369) (end 94.08 59.1369) (width 0.25) (layer "F.Cu") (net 14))
 (segment (start 97 130) (end 97 62.0569) (width 0.25) (layer "F.Cu") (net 15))
 (segment (start 96.62 60.5) (end 96.62 61.6769) (width 0.25) (layer "F.Cu") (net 15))
 (segment (start 97 62.0569) (end 96.62 61.6769) (width 0.25) (layer "F.Cu") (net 15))
 (segment (start 96.62 57.96) (end 96.62 59.1369) (width 0.25) (layer "F.Cu") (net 16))
 (segment (start 98.5 130) (end 97.89 129.39) (width 0.25) (layer "F.Cu") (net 16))
 (segment (start 97.89 60.0411) (end 96.9858 59.1369) (width 0.25) (layer "F.Cu") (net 16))
 (segment (start 97.89 129.39) (end 97.89 60.0411) (width 0.25) (layer "F.Cu") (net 16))
 (segment (start 96.9858 59.1369) (end 96.62 59.1369) (width 0.25) (layer "F.Cu") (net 16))
 (segment (start 98.6619 62.175) (end 99.16 61.6769) (width 0.25) (layer "F.Cu") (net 17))
 (segment (start 99.16 60.5) (end 99.16 61.6769) (width 0.25) (layer "F.Cu") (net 17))
 (segment (start 100 130) (end 100 114.506) (width 0.25) (layer "F.Cu") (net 17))
 (segment (start 100 114.506) (end 98.6619 113.1679) (width 0.25) (layer "F.Cu") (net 17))
 (segment (start 98.6619 113.1679) (end 98.6619 62.175) (width 0.25) (layer "F.Cu") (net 17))
 (segment (start 100.43 60.0411) (end 99.5258 59.1369) (width 0.25) (layer "F.Cu") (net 18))
 (segment (start 99.16 57.96) (end 99.16 59.1369) (width 0.25) (layer "F.Cu") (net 18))
 (segment (start 101.5 99.1835) (end 100.43 98.1135) (width 0.25) (layer "F.Cu") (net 18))
 (segment (start 99.5258 59.1369) (end 99.16 59.1369) (width 0.25) (layer "F.Cu") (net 18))
 (segment (start 100.43 98.1135) (end 100.43 60.0411) (width 0.25) (layer "F.Cu") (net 18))
 (segment (start 101.5 130) (end 101.5 99.1835) (width 0.25) (layer "F.Cu") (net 18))
 (segment (start 101.7 97.8537) (end 101.7 60.5) (width 0.25) (layer "F.Cu") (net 19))
 (segment (start 103 130) (end 102.5196 129.5196) (width 0.25) (layer "F.Cu") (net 19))
 (segment (start 102.5196 98.6733) (end 101.7 97.8537) (width 0.25) (layer "F.Cu") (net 19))
 (segment (start 102.5196 129.5196) (end 102.5196 98.6733) (width 0.25) (layer "F.Cu") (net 19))
 (segment (start 103.4219 125.3059) (end 103.4219 98.7112) (width 0.25) (layer "F.Cu") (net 20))
 (segment (start 102.0658 59.1369) (end 101.7 59.1369) (width 0.25) (layer "F.Cu") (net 20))
 (segment (start 104.5 130) (end 104.5 126.384) (width 0.25) (layer "F.Cu") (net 20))
 (segment (start 102.97 60.0411) (end 102.0658 59.1369) (width 0.25) (layer "F.Cu") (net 20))
 (segment (start 104.5 126.384) (end 103.4219 125.3059) (width 0.25) (layer "F.Cu") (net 20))
 (segment (start 103.4219 98.7112) (end 102.97 98.2593) (width 0.25) (layer "F.Cu") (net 20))
 (segment (start 101.7 57.96) (end 101.7 59.1369) (width 0.25) (layer "F.Cu") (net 20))
 (segment (start 102.97 98.2593) (end 102.97 60.0411) (width 0.25) (layer "F.Cu") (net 20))
 (segment (start 104.24 123.5607) (end 104.24 60.5) (width 0.25) (layer "F.Cu") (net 21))
 (segment (start 106 125.3207) (end 104.24 123.5607) (width 0.25) (layer "F.Cu") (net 21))
 (segment (start 106 130) (end 106 125.3207) (width 0.25) (layer "F.Cu") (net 21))
 (segment (start 107.5 130) (end 107.5 124.6611) (width 0.25) (layer "F.Cu") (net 22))
 (segment (start 104.24 57.96) (end 104.24 59.1369) (width 0.25) (layer "F.Cu") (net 22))
 (segment (start 104.6058 59.1369) (end 104.24 59.1369) (width 0.25) (layer "F.Cu") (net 22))
 (segment (start 107.5 124.6611) (end 105.51 122.6711) (width 0.25) (layer "F.Cu") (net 22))
 (segment (start 105.51 122.6711) (end 105.51 60.0411) (width 0.25) (layer "F.Cu") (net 22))
 (segment (start 105.51 60.0411) (end 104.6058 59.1369) (width 0.25) (layer "F.Cu") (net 22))
 (segment (start 109 122.5852) (end 106.78 120.3652) (width 0.25) (layer "F.Cu") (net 23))
 (segment (start 109 130) (end 109 122.5852) (width 0.25) (layer "F.Cu") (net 23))
 (segment (start 106.78 120.3652) (end 106.78 60.5) (width 0.25) (layer "F.Cu") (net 23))
 (segment (start 110.5 130) (end 110.5 123.3911) (width 0.25) (layer "F.Cu") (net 24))
 (segment (start 110.5 123.3911) (end 108.05 120.9411) (width 0.25) (layer "F.Cu") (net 24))
 (segment (start 106.78 57.96) (end 106.78 59.1369) (width 0.25) (layer "F.Cu") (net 24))
 (segment (start 108.05 60.0411) (end 107.1458 59.1369) (width 0.25) (layer "F.Cu") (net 24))
 (segment (start 108.05 120.9411) (end 108.05 60.0411) (width 0.25) (layer "F.Cu") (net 24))
 (segment (start 107.1458 59.1369) (end 106.78 59.1369) (width 0.25) (layer "F.Cu") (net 24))
 (segment (start 109.32 121.2538) (end 109.32 61.6769) (width 0.25) (layer "F.Cu") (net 25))
 (segment (start 112 130) (end 112 123.9338) (width 0.25) (layer "F.Cu") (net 25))
 (segment (start 109.32 60.5) (end 109.32 61.6769) (width 0.25) (layer "F.Cu") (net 25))
 (segment (start 112 123.9338) (end 109.32 121.2538) (width 0.25) (layer "F.Cu") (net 25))
 (segment (start 110.59 60.0411) (end 109.6858 59.1369) (width 0.25) (layer "F.Cu") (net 26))
 (segment (start 113.5 124.7946) (end 110.59 121.8846) (width 0.25) (layer "F.Cu") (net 26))
 (segment (start 109.6858 59.1369) (end 109.32 59.1369) (width 0.25) (layer "F.Cu") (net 26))
 (segment (start 113.5 130) (end 113.5 124.7946) (width 0.25) (layer "F.Cu") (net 26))
 (segment (start 110.59 121.8846) (end 110.59 60.0411) (width 0.25) (layer "F.Cu") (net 26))
 (segment (start 109.32 57.96) (end 109.32 59.1369) (width 0.25) (layer "F.Cu") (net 26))
 (segment (start 115 130) (end 115 125.6555) (width 0.25) (layer "F.Cu") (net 27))
 (segment (start 115 125.6555) (end 111.86 122.5155) (width 0.25) (layer "F.Cu") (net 27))
 (segment (start 111.86 122.5155) (end 111.86 60.5) (width 0.25) (layer "F.Cu") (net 27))
 (segment (start 111.86 57.96) (end 111.86 59.1369) (width 0.25) (layer "F.Cu") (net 28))
 (segment (start 116.5 125.0346) (end 113.13 121.6646) (width 0.25) (layer "F.Cu") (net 28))
 (segment (start 116.5 130) (end 116.5 125.0346) (width 0.25) (layer "F.Cu") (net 28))
 (segment (start 113.13 60.0411) (end 112.2258 59.1369) (width 0.25) (layer "F.Cu") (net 28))
 (segment (start 113.13 121.6646) (end 113.13 60.0411) (width 0.25) (layer "F.Cu") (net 28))
 (segment (start 112.2258 59.1369) (end 111.86 59.1369) (width 0.25) (layer "F.Cu") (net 28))
 (segment (start 118 125.4415) (end 114.4 121.8415) (width 0.25) (layer "F.Cu") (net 29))
 (segment (start 118 130) (end 118 125.4415) (width 0.25) (layer "F.Cu") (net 29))
 (segment (start 114.4 121.8415) (end 114.4 60.5) (width 0.25) (layer "F.Cu") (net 29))
 (segment (start 119.5 97.4605) (end 115.67 93.6305) (width 0.25) (layer "F.Cu") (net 30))
 (segment (start 114.4 57.96) (end 114.4 59.1369) (width 0.25) (layer "F.Cu") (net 30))
 (segment (start 114.7658 59.1369) (end 114.4 59.1369) (width 0.25) (layer "F.Cu") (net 30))
 (segment (start 115.67 60.0411) (end 114.7658 59.1369) (width 0.25) (layer "F.Cu") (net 30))
 (segment (start 115.67 93.6305) (end 115.67 60.0411) (width 0.25) (layer "F.Cu") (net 30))
 (segment (start 119.5 130) (end 119.5 97.4605) (width 0.25) (layer "F.Cu") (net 30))
 (segment (start 121 130) (end 121 96.1085) (width 0.25) (layer "F.Cu") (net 31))
 (segment (start 116.94 92.0485) (end 116.94 60.5) (width 0.25) (layer "F.Cu") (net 31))
 (segment (start 121 96.1085) (end 116.94 92.0485) (width 0.25) (layer "F.Cu") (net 31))
 (segment (start 116.94 59.1369) (end 117.3079 59.1369) (width 0.25) (layer "F.Cu") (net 32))
 (segment (start 122.5 96.0914) (end 122.5 130) (width 0.25) (layer "F.Cu") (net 32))
 (segment (start 117.3079 59.1369) (end 118.1169 59.9459) (width 0.25) (layer "F.Cu") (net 32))
 (segment (start 116.94 57.96) (end 116.94 59.1369) (width 0.25) (layer "F.Cu") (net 32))
 (segment (start 118.1169 59.9459) (end 118.1169 91.7083) (width 0.25) (layer "F.Cu") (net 32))
 (segment (start 118.1169 91.7083) (end 122.5 96.0914) (width 0.25) (layer "F.Cu") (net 32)))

